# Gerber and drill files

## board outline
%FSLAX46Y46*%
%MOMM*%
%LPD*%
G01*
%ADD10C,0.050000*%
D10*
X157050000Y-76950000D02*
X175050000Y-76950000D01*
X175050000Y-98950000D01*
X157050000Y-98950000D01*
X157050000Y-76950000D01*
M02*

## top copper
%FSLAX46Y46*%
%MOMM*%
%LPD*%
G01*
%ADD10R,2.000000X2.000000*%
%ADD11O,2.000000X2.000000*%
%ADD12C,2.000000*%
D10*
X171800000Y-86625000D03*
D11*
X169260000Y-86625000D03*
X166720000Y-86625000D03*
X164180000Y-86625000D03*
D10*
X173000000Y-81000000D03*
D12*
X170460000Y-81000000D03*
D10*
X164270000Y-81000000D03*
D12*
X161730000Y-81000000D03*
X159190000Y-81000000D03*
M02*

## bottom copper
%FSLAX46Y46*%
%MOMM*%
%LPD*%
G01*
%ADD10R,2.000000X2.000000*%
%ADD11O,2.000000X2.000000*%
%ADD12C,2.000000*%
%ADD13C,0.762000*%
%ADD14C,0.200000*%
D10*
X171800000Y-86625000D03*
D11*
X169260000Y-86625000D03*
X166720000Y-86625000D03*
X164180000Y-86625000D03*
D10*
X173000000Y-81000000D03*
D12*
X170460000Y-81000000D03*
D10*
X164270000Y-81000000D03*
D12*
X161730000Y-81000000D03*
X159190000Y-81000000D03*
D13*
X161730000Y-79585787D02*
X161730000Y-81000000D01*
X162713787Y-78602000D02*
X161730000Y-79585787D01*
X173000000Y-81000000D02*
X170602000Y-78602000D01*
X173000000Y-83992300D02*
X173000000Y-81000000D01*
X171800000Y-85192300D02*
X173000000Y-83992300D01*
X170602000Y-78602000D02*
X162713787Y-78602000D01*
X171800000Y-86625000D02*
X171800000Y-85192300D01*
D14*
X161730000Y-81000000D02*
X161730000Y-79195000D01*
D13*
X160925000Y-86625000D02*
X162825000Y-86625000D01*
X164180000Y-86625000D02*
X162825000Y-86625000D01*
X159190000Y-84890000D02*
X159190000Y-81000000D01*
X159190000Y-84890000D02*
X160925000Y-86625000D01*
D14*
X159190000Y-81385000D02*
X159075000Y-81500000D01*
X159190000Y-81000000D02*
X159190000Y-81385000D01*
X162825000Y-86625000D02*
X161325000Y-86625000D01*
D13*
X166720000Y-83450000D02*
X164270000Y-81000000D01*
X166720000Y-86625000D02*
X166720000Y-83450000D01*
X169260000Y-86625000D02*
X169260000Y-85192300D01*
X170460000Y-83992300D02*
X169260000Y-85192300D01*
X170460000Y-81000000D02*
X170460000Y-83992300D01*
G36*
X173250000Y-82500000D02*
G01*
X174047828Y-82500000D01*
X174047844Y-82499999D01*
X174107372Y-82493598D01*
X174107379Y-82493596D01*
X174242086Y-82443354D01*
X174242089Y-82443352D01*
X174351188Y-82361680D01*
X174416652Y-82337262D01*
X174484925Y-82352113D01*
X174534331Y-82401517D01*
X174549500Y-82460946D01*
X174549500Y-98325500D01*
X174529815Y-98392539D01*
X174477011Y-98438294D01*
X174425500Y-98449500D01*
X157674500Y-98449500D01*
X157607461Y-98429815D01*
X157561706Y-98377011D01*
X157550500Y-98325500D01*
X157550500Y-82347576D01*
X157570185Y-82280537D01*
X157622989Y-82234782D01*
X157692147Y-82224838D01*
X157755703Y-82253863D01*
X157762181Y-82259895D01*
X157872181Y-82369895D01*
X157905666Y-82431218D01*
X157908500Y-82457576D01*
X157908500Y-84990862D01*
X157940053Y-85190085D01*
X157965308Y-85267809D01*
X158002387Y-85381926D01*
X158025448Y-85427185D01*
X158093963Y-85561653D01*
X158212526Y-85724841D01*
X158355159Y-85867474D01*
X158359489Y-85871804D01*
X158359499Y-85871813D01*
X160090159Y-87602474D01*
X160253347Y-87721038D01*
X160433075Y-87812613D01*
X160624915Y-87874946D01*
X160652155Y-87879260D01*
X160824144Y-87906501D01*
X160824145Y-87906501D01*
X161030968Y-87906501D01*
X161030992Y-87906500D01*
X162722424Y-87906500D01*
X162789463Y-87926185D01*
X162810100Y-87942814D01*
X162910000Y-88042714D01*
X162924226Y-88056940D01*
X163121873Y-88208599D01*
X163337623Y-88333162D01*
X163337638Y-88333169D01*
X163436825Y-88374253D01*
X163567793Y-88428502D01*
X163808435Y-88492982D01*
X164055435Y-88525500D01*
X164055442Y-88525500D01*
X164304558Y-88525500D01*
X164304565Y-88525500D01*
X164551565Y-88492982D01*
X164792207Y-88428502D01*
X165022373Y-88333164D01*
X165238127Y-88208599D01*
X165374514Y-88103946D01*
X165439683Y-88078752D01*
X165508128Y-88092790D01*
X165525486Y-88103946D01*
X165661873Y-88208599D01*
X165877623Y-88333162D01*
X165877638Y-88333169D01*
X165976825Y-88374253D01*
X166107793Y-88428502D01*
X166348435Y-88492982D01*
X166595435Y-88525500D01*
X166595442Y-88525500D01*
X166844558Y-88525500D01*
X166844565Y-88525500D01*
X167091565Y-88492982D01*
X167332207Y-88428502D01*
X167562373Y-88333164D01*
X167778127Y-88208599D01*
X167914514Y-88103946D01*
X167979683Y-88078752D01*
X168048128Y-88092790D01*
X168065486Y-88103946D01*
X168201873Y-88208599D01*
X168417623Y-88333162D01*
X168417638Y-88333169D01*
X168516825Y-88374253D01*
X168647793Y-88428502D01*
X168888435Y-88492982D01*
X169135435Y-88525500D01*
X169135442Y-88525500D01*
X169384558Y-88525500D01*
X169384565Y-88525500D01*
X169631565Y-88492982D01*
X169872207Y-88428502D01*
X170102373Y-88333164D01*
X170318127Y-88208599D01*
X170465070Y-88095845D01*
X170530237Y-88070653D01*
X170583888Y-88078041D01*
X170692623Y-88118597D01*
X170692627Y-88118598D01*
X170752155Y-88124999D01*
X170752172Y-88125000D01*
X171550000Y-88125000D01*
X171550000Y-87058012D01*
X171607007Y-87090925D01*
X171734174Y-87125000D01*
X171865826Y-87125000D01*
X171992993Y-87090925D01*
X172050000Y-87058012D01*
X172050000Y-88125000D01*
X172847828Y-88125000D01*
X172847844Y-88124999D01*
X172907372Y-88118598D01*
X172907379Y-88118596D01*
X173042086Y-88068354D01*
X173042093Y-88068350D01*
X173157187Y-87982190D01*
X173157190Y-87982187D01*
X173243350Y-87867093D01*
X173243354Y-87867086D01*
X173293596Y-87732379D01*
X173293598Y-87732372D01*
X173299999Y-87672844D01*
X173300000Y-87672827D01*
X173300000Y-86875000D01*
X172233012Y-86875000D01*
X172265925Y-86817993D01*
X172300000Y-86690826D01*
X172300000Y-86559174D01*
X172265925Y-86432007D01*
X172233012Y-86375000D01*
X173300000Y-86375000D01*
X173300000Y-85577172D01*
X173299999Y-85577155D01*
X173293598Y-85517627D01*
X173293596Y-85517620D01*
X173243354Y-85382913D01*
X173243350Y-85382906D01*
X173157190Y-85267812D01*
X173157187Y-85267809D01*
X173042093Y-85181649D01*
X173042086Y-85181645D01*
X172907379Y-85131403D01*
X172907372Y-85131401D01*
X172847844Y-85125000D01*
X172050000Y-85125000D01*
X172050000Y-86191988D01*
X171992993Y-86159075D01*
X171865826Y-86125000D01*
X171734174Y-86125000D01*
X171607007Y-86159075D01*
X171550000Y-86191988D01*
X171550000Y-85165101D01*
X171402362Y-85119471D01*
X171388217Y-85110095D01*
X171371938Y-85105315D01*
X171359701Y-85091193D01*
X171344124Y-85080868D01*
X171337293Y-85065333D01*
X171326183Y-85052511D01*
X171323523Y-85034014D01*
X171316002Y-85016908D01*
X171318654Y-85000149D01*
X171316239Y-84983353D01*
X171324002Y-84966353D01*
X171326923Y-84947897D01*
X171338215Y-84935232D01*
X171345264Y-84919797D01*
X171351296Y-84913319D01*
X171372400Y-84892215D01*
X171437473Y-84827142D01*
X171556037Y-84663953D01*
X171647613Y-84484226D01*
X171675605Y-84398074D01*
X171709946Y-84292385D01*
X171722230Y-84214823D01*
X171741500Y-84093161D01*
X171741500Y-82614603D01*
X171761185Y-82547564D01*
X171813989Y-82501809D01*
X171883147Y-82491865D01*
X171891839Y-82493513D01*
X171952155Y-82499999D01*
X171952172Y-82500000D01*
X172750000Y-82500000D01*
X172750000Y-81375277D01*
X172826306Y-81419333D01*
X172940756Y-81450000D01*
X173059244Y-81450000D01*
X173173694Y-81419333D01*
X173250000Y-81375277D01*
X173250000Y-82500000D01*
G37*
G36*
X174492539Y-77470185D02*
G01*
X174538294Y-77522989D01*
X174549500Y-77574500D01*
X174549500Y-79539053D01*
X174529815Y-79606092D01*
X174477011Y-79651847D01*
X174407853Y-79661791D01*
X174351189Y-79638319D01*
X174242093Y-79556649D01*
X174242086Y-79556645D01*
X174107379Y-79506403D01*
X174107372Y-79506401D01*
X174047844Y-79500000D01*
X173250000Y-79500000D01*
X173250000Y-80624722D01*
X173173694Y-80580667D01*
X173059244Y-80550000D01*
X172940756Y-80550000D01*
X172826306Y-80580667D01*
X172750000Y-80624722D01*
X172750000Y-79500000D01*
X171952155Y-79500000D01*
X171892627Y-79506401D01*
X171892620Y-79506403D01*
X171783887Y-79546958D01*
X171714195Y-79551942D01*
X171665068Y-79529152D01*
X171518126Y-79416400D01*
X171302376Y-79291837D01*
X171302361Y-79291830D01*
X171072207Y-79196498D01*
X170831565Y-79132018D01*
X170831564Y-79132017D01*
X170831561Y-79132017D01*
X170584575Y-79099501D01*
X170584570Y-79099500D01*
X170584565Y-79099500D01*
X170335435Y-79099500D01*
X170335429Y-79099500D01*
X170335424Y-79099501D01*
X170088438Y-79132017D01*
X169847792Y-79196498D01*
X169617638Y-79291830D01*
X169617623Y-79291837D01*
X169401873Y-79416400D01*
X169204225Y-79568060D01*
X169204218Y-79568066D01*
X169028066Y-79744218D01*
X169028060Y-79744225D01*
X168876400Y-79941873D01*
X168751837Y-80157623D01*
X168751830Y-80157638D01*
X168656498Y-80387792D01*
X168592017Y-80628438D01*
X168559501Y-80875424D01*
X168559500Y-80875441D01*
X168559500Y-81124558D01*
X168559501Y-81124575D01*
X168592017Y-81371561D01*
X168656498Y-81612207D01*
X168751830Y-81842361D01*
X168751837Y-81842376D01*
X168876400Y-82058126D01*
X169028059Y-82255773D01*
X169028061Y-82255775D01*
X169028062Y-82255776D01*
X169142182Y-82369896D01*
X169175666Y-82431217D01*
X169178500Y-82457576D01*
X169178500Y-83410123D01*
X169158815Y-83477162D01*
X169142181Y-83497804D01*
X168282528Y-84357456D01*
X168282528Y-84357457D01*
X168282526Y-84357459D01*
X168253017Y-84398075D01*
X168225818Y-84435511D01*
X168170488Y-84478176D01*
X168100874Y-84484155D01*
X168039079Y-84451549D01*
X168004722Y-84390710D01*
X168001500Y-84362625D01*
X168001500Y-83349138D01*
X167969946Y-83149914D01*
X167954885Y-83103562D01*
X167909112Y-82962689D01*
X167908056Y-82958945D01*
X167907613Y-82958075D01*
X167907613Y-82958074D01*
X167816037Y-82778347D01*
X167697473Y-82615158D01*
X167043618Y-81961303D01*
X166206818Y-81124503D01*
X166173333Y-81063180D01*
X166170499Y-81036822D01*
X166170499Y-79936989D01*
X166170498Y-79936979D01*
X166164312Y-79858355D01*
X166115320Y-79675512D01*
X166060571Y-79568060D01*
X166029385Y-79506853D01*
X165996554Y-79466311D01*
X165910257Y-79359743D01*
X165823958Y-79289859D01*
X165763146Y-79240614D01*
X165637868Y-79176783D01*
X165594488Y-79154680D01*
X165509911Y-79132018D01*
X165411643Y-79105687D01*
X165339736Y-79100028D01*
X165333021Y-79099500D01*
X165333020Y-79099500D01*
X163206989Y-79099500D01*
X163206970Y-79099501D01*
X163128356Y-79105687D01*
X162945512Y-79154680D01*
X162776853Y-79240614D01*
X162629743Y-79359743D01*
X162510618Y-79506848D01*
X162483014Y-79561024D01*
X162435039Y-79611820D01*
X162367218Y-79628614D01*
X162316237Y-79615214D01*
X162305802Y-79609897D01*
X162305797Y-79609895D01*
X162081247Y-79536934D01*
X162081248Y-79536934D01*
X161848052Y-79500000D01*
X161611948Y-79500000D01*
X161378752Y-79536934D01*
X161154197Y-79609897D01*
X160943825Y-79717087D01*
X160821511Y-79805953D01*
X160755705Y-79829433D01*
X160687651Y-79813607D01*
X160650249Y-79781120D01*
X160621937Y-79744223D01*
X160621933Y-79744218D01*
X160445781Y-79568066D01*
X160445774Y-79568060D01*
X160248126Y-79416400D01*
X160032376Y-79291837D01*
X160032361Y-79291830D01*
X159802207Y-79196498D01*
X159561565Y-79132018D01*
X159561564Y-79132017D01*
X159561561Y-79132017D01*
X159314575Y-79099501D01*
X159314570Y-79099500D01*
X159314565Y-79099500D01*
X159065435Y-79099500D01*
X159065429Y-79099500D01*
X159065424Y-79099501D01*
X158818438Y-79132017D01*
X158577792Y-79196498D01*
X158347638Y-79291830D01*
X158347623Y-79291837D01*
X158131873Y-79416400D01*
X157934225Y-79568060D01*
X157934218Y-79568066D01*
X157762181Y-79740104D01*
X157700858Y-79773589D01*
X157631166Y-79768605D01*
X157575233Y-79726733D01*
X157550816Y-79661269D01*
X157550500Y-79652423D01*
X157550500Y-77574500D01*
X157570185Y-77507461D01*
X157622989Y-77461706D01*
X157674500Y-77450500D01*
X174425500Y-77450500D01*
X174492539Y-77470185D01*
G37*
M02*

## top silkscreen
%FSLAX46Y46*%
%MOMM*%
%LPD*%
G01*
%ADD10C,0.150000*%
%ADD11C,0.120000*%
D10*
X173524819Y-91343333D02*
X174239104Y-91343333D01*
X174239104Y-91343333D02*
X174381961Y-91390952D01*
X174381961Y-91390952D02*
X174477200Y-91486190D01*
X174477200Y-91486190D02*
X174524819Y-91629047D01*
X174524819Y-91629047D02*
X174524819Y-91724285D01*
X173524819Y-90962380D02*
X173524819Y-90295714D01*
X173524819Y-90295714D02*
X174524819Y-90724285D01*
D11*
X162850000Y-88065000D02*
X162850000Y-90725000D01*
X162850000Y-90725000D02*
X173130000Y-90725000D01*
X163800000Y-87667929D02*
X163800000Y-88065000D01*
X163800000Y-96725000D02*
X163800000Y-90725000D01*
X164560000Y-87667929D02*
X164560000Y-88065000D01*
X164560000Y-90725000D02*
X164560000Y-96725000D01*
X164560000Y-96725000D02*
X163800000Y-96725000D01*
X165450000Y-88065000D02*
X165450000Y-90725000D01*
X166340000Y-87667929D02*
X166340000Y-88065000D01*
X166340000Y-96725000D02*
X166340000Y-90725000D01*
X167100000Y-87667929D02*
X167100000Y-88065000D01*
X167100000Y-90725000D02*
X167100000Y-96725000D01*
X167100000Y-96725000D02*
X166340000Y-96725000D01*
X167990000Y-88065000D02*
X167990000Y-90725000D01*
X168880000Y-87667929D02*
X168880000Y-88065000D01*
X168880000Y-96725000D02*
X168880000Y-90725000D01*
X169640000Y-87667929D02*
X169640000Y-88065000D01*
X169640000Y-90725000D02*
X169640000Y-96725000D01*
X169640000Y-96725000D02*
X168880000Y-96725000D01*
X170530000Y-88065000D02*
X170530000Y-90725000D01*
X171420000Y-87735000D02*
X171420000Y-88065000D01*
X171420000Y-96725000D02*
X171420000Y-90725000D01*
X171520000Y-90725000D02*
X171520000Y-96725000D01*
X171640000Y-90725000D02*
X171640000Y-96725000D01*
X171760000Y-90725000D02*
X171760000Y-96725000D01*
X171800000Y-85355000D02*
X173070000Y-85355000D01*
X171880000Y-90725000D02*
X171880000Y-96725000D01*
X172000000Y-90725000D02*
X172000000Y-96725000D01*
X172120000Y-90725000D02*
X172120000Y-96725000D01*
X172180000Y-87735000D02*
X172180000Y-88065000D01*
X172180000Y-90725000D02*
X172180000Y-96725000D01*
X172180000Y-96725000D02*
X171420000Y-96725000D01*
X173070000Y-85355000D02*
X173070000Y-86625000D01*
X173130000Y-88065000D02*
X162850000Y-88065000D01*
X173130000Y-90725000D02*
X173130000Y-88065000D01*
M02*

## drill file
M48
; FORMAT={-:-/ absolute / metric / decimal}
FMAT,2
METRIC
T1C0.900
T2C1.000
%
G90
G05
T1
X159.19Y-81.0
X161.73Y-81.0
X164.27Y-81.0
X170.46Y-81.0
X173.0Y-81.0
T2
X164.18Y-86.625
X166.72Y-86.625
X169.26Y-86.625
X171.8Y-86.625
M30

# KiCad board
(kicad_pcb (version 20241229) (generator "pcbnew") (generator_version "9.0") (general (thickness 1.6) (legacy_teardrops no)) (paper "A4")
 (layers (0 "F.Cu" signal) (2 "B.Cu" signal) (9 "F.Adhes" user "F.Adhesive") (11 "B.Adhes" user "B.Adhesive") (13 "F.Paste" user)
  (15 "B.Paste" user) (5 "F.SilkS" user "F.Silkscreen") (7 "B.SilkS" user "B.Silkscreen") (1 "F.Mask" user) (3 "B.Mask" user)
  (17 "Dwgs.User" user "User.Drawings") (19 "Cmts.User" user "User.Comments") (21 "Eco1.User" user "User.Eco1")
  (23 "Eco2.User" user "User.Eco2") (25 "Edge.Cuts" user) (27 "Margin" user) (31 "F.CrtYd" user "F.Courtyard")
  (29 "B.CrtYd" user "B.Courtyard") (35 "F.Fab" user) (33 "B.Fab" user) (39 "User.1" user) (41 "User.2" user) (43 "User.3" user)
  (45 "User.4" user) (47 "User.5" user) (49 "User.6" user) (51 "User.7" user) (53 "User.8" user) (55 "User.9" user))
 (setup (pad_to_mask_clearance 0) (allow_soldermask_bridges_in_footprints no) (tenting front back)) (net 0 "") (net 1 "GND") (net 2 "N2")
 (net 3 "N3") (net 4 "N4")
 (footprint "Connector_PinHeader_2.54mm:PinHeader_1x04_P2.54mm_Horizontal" (layer "F.Cu") (at 171.8 86.625 -90)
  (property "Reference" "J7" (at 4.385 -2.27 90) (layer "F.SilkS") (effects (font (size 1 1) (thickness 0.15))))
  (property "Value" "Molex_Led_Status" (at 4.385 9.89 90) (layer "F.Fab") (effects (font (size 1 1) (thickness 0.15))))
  (fp_line (start 1.44 8.95) (end 4.1 8.95) (stroke (width 0.12) (type solid)) (layer "F.SilkS"))
  (fp_line (start 4.1 8.95) (end 4.1 -1.33) (stroke (width 0.12) (type solid)) (layer "F.SilkS"))
  (fp_line (start 1.042929 8) (end 1.44 8) (stroke (width 0.12) (type solid)) (layer "F.SilkS"))
  (fp_line (start 10.1 8) (end 4.1 8) (stroke (width 0.12) (type solid)) (layer "F.SilkS"))
  (fp_line (start 1.042929 7.24) (end 1.44 7.24) (stroke (width 0.12) (type solid)) (layer "F.SilkS"))
  (fp_line (start 4.1 7.24) (end 10.1 7.24) (stroke (width 0.12) (type solid)) (layer "F.SilkS"))
  (fp_line (start 10.1 7.24) (end 10.1 8) (stroke (width 0.12) (type solid)) (layer "F.SilkS"))
  (fp_line (start 1.44 6.35) (end 4.1 6.35) (stroke (width 0.12) (type solid)) (layer "F.SilkS"))
  (fp_line (start 1.042929 5.46) (end 1.44 5.46) (stroke (width 0.12) (type solid)) (layer "F.SilkS"))
  (fp_line (start 10.1 5.46) (end 4.1 5.46) (stroke (width 0.12) (type solid)) (layer "F.SilkS"))
  (fp_line (start 1.042929 4.7) (end 1.44 4.7) (stroke (width 0.12) (type solid)) (layer "F.SilkS"))
  (fp_line (start 4.1 4.7) (end 10.1 4.7) (stroke (width 0.12) (type solid)) (layer "F.SilkS"))
  (fp_line (start 10.1 4.7) (end 10.1 5.46) (stroke (width 0.12) (type solid)) (layer "F.SilkS"))
  (fp_line (start 1.44 3.81) (end 4.1 3.81) (stroke (width 0.12) (type solid)) (layer "F.SilkS"))
  (fp_line (start 1.042929 2.92) (end 1.44 2.92) (stroke (width 0.12) (type solid)) (layer "F.SilkS"))
  (fp_line (start 10.1 2.92) (end 4.1 2.92) (stroke (width 0.12) (type solid)) (layer "F.SilkS"))
  (fp_line (start 1.042929 2.16) (end 1.44 2.16) (stroke (width 0.12) (type solid)) (layer "F.SilkS"))
  (fp_line (start 4.1 2.16) (end 10.1 2.16) (stroke (width 0.12) (type solid)) (layer "F.SilkS"))
  (fp_line (start 10.1 2.16) (end 10.1 2.92) (stroke (width 0.12) (type solid)) (layer "F.SilkS"))
  (fp_line (start 1.44 1.27) (end 4.1 1.27) (stroke (width 0.12) (type solid)) (layer "F.SilkS"))
  (fp_line (start 1.11 0.38) (end 1.44 0.38) (stroke (width 0.12) (type solid)) (layer "F.SilkS"))
  (fp_line (start 10.1 0.38) (end 4.1 0.38) (stroke (width 0.12) (type solid)) (layer "F.SilkS"))
  (fp_line (start 4.1 0.28) (end 10.1 0.28) (stroke (width 0.12) (type solid)) (layer "F.SilkS"))
  (fp_line (start 4.1 0.16) (end 10.1 0.16) (stroke (width 0.12) (type solid)) (layer "F.SilkS"))
  (fp_line (start 4.1 0.04) (end 10.1 0.04) (stroke (width 0.12) (type solid)) (layer "F.SilkS"))
  (fp_line (start -1.27 0) (end -1.27 -1.27) (stroke (width 0.12) (type solid)) (layer "F.SilkS"))
  (fp_line (start 4.1 -0.08) (end 10.1 -0.08) (stroke (width 0.12) (type solid)) (layer "F.SilkS"))
  (fp_line (start 4.1 -0.2) (end 10.1 -0.2) (stroke (width 0.12) (type solid)) (layer "F.SilkS"))
  (fp_line (start 4.1 -0.32) (end 10.1 -0.32) (stroke (width 0.12) (type solid)) (layer "F.SilkS"))
  (fp_line (start 1.11 -0.38) (end 1.44 -0.38) (stroke (width 0.12) (type solid)) (layer "F.SilkS"))
  (fp_line (start 4.1 -0.38) (end 10.1 -0.38) (stroke (width 0.12) (type solid)) (layer "F.SilkS"))
  (fp_line (start 10.1 -0.38) (end 10.1 0.38) (stroke (width 0.12) (type solid)) (layer "F.SilkS"))
  (fp_line (start -1.27 -1.27) (end 0 -1.27) (stroke (width 0.12) (type solid)) (layer "F.SilkS"))
  (fp_line (start 1.44 -1.33) (end 1.44 8.95) (stroke (width 0.12) (type solid)) (layer "F.SilkS"))
  (fp_line (start 4.1 -1.33) (end 1.44 -1.33) (stroke (width 0.12) (type solid)) (layer "F.SilkS"))
  (pad "1" thru_hole rect (at 0 0 270) (size 2 2) (drill 1) (layers "*.Cu" "*.Mask") (remove_unused_layers no) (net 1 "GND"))
  (pad "2" thru_hole oval (at 0 2.54 270) (size 2 2) (drill 1) (layers "*.Cu" "*.Mask") (remove_unused_layers no) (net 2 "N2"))
  (pad "3" thru_hole oval (at 0 5.08 270) (size 2 2) (drill 1) (layers "*.Cu" "*.Mask") (remove_unused_layers no) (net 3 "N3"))
  (pad "4" thru_hole oval (at 0 7.62 270) (size 2 2) (drill 1) (layers "*.Cu" "*.Mask") (remove_unused_layers no) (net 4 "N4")))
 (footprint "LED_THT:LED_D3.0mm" (layer "B.Cu") (at 173 81 180)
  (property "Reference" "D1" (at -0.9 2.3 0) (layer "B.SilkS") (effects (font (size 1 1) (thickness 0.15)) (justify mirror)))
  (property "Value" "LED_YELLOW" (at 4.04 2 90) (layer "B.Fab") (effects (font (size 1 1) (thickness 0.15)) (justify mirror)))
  (pad "1" thru_hole rect (at 0 0 180) (size 2 2) (drill 0.9) (layers "*.Cu" "*.Mask") (remove_unused_layers no) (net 1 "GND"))
  (pad "2" thru_hole circle (at 2.54 0 180) (size 2 2) (drill 0.9) (layers "*.Cu" "*.Mask") (remove_unused_layers no) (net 2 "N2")))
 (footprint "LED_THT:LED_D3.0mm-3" (layer "B.Cu") (at 164.27 81 180)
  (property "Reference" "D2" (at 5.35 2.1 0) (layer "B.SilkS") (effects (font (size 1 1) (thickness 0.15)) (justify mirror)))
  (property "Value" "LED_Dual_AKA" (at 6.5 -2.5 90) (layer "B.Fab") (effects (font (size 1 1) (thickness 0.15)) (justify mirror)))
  (pad "1" thru_hole rect (at 0 0 180) (size 2 2) (drill 0.9) (layers "*.Cu" "*.Mask") (remove_unused_layers no) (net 3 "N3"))
  (pad "2" thru_hole circle (at 2.54 0 180) (size 2 2) (drill 0.9) (layers "*.Cu" "*.Mask") (remove_unused_layers no) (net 1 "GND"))
  (pad "3" thru_hole circle (at 5.08 0 180) (size 2 2) (drill 0.9) (layers "*.Cu" "*.Mask") (remove_unused_layers no) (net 4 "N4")))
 (gr_rect (start 157.05 76.95) (end 175.05 98.95) (stroke (width 0.05) (type solid)) (fill no) (layer "Edge.Cuts"))
 (segment (start 161.73 79.585787) (end 161.73 81) (width 0.762) (layer "B.Cu") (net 1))
 (segment (start 162.713787 78.602) (end 161.73 79.585787) (width 0.762) (layer "B.Cu") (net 1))
 (segment (start 173 81) (end 170.602 78.602) (width 0.762) (layer "B.Cu") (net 1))
 (segment (start 173 83.9923) (end 173 81) (width 0.762) (layer "B.Cu") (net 1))
 (segment (start 171.8 85.1923) (end 173 83.9923) (width 0.762) (layer "B.Cu") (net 1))
 (segment (start 170.602 78.602) (end 162.713787 78.602) (width 0.762) (layer "B.Cu") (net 1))
 (segment (start 171.8 86.625) (end 171.8 85.1923) (width 0.762) (layer "B.Cu") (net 1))
 (segment (start 161.73 81) (end 161.73 79.195) (width 0.2) (layer "B.Cu") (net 1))
 (segment (start 160.925 86.625) (end 162.825 86.625) (width 0.762) (layer "B.Cu") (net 4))
 (segment (start 164.18 86.625) (end 162.825 86.625) (width 0.762) (layer "B.Cu") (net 4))
 (segment (start 159.19 84.89) (end 159.19 81) (width 0.762) (layer "B.Cu") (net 4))
 (segment (start 159.19 84.89) (end 160.925 86.625) (width 0.762) (layer "B.Cu") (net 4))
 (segment (start 159.19 81.385) (end 159.075 81.5) (width 0.2) (layer "B.Cu") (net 4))
 (segment (start 159.19 81) (end 159.19 81.385) (width 0.2) (layer "B.Cu") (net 4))
 (segment (start 162.825 86.625) (end 161.325 86.625) (width 0.2) (layer "B.Cu") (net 4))
 (segment (start 166.72 83.45) (end 164.27 81) (width 0.762) (layer "B.Cu") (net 3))
 (segment (start 166.72 86.625) (end 166.72 83.45) (width 0.762) (layer "B.Cu") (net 3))
 (segment (start 169.26 86.625) (end 169.26 85.1923) (width 0.762) (layer "B.Cu") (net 2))
 (segment (start 170.46 83.9923) (end 169.26 85.1923) (width 0.762) (layer "B.Cu") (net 2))
 (segment (start 170.46 81) (end 170.46 83.9923) (width 0.762) (layer "B.Cu") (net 2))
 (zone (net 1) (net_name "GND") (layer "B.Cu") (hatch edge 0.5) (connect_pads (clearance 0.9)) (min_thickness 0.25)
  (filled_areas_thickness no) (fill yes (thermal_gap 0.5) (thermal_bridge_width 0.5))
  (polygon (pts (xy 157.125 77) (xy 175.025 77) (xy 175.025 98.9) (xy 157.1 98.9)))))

